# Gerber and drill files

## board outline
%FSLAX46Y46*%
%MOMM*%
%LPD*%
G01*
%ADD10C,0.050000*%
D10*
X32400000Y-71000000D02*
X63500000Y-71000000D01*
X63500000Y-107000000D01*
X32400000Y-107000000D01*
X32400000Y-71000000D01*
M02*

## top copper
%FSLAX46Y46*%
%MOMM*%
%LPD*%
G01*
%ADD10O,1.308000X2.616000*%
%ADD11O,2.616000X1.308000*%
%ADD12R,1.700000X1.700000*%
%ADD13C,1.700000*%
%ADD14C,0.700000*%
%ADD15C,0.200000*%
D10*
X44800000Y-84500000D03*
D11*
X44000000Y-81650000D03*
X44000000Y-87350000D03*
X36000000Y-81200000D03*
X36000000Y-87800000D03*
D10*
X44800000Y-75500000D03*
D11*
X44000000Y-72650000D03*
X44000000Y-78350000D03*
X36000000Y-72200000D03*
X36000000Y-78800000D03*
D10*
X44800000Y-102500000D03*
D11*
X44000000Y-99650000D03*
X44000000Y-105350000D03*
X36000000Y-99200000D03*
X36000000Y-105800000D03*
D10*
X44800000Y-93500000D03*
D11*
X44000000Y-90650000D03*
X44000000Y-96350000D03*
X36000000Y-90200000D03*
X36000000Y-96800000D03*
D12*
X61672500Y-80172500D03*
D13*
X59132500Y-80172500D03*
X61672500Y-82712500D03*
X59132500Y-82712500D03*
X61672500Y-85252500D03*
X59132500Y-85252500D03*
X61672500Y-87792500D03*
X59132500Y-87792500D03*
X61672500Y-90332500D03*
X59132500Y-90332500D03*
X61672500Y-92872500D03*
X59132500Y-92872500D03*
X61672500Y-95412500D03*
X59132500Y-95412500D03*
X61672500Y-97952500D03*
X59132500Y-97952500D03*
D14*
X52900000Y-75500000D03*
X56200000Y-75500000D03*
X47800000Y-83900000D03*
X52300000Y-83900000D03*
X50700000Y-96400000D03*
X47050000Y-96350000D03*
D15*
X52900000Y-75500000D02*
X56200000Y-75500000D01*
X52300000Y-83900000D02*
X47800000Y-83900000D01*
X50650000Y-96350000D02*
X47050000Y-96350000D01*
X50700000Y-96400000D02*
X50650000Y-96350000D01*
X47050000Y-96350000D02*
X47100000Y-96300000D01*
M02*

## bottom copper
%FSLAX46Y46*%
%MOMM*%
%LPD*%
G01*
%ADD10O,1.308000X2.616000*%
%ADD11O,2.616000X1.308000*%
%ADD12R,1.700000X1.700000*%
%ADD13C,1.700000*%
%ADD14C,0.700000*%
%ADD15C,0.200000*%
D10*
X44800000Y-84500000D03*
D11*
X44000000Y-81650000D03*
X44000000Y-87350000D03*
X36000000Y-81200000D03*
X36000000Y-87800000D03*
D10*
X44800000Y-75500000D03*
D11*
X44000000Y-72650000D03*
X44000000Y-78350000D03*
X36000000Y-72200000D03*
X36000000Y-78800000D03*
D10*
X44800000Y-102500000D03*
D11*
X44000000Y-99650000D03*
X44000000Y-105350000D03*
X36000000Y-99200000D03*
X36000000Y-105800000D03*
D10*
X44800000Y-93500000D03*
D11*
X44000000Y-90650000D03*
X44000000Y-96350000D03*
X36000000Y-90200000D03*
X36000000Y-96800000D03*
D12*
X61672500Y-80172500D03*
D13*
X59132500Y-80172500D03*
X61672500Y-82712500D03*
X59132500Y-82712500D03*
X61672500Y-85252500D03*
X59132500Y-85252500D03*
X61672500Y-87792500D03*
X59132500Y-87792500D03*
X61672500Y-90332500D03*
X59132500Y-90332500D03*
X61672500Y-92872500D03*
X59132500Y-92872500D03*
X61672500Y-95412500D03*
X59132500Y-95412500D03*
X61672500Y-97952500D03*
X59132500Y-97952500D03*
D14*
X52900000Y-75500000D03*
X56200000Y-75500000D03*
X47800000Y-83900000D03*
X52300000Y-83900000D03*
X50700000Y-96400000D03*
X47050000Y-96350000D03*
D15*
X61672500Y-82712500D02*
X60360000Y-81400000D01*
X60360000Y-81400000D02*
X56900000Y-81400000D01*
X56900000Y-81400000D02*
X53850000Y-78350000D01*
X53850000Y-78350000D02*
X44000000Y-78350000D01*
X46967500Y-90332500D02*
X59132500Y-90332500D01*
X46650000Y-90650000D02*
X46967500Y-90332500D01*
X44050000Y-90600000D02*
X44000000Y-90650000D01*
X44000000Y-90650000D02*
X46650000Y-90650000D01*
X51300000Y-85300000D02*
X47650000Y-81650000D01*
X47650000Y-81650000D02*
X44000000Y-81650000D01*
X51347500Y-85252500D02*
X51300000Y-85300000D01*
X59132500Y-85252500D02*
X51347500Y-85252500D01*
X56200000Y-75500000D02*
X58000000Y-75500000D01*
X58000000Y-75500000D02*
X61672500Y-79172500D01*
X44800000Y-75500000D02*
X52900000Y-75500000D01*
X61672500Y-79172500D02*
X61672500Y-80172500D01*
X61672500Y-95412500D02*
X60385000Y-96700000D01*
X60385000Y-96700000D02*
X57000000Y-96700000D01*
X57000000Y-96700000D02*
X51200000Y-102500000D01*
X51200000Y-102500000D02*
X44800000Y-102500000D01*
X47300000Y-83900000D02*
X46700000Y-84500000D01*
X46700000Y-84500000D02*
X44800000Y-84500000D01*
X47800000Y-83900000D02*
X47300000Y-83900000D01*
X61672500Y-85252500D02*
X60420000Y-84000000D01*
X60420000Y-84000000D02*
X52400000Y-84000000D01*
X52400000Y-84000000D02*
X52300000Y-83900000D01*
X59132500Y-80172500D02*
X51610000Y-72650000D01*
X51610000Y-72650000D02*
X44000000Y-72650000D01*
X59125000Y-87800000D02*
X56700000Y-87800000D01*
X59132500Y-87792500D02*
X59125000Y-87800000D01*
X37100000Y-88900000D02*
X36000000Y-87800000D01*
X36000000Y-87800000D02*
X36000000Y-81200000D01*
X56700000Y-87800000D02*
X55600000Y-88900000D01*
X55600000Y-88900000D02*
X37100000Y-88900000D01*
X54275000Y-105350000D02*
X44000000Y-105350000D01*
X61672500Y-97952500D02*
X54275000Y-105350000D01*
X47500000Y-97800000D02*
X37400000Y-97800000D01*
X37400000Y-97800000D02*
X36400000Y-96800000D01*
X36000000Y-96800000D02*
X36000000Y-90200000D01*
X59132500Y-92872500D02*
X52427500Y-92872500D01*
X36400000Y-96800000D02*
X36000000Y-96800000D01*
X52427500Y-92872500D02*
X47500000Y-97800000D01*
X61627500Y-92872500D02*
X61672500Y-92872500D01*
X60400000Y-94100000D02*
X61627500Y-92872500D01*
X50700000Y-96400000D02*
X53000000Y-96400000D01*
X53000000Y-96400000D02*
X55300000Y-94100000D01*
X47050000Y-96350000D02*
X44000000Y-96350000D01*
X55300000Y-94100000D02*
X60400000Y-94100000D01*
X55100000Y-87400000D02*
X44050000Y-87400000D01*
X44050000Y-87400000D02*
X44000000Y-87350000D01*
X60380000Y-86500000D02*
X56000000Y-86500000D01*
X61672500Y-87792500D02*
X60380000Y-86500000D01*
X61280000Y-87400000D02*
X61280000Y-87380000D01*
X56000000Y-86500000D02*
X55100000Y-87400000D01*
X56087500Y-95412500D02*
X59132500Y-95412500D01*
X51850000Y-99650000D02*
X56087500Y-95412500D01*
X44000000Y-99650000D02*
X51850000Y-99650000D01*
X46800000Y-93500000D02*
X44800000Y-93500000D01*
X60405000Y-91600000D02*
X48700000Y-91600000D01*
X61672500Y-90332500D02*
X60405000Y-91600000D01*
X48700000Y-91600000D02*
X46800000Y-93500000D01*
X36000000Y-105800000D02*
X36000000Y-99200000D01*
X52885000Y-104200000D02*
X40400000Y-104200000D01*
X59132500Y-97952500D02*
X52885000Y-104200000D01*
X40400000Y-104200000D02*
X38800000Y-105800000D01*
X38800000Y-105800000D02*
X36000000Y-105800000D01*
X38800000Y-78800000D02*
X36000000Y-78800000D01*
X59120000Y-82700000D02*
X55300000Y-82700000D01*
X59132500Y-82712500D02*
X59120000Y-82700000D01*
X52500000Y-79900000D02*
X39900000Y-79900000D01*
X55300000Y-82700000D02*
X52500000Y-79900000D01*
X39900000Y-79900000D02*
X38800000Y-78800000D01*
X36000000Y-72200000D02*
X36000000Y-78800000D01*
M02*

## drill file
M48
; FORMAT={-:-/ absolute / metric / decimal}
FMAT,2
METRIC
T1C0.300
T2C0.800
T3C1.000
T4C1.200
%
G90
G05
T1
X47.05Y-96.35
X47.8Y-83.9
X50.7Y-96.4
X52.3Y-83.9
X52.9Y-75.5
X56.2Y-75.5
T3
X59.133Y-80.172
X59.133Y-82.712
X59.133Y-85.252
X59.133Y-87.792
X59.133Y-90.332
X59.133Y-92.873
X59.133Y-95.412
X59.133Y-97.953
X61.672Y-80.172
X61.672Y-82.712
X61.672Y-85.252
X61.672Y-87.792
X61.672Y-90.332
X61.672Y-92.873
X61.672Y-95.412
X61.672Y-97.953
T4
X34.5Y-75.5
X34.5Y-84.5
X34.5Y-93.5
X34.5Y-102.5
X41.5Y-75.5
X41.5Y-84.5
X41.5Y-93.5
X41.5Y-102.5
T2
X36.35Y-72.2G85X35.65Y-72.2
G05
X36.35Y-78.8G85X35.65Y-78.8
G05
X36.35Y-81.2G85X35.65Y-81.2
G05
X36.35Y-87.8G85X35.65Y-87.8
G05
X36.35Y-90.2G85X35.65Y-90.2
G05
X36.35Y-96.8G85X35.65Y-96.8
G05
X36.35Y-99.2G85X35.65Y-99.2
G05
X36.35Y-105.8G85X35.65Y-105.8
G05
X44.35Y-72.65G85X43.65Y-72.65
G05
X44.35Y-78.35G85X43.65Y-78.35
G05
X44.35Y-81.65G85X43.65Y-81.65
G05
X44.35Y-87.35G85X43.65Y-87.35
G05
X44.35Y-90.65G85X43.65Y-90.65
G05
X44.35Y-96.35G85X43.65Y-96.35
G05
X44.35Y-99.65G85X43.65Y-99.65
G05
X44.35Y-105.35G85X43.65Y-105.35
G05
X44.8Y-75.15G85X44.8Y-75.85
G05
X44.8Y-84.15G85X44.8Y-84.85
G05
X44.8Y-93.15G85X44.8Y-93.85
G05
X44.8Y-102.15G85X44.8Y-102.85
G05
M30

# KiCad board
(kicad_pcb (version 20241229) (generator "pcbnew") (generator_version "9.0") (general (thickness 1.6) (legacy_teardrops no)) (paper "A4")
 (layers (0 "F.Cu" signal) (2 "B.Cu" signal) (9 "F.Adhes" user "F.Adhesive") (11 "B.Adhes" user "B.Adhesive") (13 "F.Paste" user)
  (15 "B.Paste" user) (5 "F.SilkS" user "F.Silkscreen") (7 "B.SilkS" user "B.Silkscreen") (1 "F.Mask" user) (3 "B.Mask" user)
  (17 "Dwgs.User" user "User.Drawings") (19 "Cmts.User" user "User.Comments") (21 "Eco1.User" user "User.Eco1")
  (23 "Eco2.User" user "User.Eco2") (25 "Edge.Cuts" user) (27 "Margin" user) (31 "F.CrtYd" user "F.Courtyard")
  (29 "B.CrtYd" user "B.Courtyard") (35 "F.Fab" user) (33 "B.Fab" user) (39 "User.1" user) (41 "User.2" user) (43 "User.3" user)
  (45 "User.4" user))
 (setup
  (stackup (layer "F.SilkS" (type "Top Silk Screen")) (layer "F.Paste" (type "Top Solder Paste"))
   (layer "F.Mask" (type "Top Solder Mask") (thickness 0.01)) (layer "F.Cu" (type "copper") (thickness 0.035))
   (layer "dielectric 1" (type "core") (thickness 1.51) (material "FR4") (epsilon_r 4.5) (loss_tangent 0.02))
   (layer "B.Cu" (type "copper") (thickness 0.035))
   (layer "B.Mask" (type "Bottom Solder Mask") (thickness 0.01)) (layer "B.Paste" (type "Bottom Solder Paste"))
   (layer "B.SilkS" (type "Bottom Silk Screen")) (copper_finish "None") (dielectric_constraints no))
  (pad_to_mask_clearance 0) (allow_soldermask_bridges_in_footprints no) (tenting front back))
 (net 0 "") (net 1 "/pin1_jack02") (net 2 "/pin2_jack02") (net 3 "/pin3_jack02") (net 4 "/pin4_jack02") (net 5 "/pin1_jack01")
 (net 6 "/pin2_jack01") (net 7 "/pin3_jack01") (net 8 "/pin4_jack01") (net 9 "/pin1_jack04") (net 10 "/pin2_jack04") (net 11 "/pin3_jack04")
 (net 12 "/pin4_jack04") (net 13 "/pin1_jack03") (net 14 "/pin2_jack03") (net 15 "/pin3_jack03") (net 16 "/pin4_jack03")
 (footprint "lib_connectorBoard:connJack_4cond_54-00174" (layer "F.Cu") (at 38 84.5 -90)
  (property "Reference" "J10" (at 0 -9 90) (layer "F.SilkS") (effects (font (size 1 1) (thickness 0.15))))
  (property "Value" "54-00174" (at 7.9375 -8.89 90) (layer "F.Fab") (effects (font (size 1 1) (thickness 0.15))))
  (pad "" np_thru_hole circle (at 0 -3.5 270) (size 1.2 1.2) (drill 1.2) (layers "*.Cu" "*.Mask"))
  (pad "" np_thru_hole circle (at 0 3.5 270) (size 1.2 1.2) (drill 1.2) (layers "*.Cu" "*.Mask"))
  (pad "1" thru_hole oval (at 0 -6.8 270) (size 2.616 1.308) (drill oval 1.5 0.8) (layers "*.Cu" "*.Mask") (remove_unused_layers no)
   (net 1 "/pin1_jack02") (solder_mask_margin 0.102))
  (pad "2" thru_hole oval (at -2.85 -6 270) (size 1.308 2.616) (drill oval 0.8 1.5) (layers "*.Cu" "*.Mask") (remove_unused_layers no)
   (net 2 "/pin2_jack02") (solder_mask_margin 0.102))
  (pad "3" thru_hole oval (at 2.85 -6 270) (size 1.308 2.616) (drill oval 0.8 1.5) (layers "*.Cu" "*.Mask") (remove_unused_layers no)
   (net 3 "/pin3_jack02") (solder_mask_margin 0.102))
  (pad "4_1" thru_hole oval (at -3.3 2 270) (size 1.308 2.616) (drill oval 0.8 1.5) (layers "*.Cu" "*.Mask") (remove_unused_layers no)
   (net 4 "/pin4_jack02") (solder_mask_margin 0.102))
  (pad "4_2" thru_hole oval (at 3.3 2 270) (size 1.308 2.616) (drill oval 0.8 1.5) (layers "*.Cu" "*.Mask") (remove_unused_layers no)
   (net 4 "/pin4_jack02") (solder_mask_margin 0.102)))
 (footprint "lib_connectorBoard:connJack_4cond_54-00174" (layer "F.Cu") (at 38 75.5 -90)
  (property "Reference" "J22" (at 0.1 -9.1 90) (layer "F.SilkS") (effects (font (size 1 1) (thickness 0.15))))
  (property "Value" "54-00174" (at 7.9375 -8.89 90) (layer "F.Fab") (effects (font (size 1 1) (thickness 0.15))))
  (pad "" np_thru_hole circle (at 0 -3.5 270) (size 1.2 1.2) (drill 1.2) (layers "*.Cu" "*.Mask"))
  (pad "" np_thru_hole circle (at 0 3.5 270) (size 1.2 1.2) (drill 1.2) (layers "*.Cu" "*.Mask"))
  (pad "1" thru_hole oval (at 0 -6.8 270) (size 2.616 1.308) (drill oval 1.5 0.8) (layers "*.Cu" "*.Mask") (remove_unused_layers no)
   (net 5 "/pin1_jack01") (solder_mask_margin 0.102))
  (pad "2" thru_hole oval (at -2.85 -6 270) (size 1.308 2.616) (drill oval 0.8 1.5) (layers "*.Cu" "*.Mask") (remove_unused_layers no)
   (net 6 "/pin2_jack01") (solder_mask_margin 0.102))
  (pad "3" thru_hole oval (at 2.85 -6 270) (size 1.308 2.616) (drill oval 0.8 1.5) (layers "*.Cu" "*.Mask") (remove_unused_layers no)
   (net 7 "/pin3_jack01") (solder_mask_margin 0.102))
  (pad "4_1" thru_hole oval (at -3.3 2 270) (size 1.308 2.616) (drill oval 0.8 1.5) (layers "*.Cu" "*.Mask") (remove_unused_layers no)
   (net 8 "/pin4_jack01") (solder_mask_margin 0.102))
  (pad "4_2" thru_hole oval (at 3.3 2 270) (size 1.308 2.616) (drill oval 0.8 1.5) (layers "*.Cu" "*.Mask") (remove_unused_layers no)
   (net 8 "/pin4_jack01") (solder_mask_margin 0.102)))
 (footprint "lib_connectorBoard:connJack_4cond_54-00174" (layer "F.Cu") (at 38 102.5 -90)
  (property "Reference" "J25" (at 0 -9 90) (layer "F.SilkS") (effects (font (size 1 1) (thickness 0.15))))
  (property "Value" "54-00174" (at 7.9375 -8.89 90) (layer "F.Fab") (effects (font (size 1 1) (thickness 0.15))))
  (pad "" np_thru_hole circle (at 0 -3.5 270) (size 1.2 1.2) (drill 1.2) (layers "*.Cu" "*.Mask"))
  (pad "" np_thru_hole circle (at 0 3.5 270) (size 1.2 1.2) (drill 1.2) (layers "*.Cu" "*.Mask"))
  (pad "1" thru_hole oval (at 0 -6.8 270) (size 2.616 1.308) (drill oval 1.5 0.8) (layers "*.Cu" "*.Mask") (remove_unused_layers no)
   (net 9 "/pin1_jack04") (solder_mask_margin 0.102))
  (pad "2" thru_hole oval (at -2.85 -6 270) (size 1.308 2.616) (drill oval 0.8 1.5) (layers "*.Cu" "*.Mask") (remove_unused_layers no)
   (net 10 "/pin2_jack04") (solder_mask_margin 0.102))
  (pad "3" thru_hole oval (at 2.85 -6 270) (size 1.308 2.616) (drill oval 0.8 1.5) (layers "*.Cu" "*.Mask") (remove_unused_layers no)
   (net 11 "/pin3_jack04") (solder_mask_margin 0.102))
  (pad "4_1" thru_hole oval (at -3.3 2 270) (size 1.308 2.616) (drill oval 0.8 1.5) (layers "*.Cu" "*.Mask") (remove_unused_layers no)
   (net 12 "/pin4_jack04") (solder_mask_margin 0.102))
  (pad "4_2" thru_hole oval (at 3.3 2 270) (size 1.308 2.616) (drill oval 0.8 1.5) (layers "*.Cu" "*.Mask") (remove_unused_layers no)
   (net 12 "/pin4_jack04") (solder_mask_margin 0.102)))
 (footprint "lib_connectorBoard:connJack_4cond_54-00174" (layer "F.Cu") (at 38 93.5 -90)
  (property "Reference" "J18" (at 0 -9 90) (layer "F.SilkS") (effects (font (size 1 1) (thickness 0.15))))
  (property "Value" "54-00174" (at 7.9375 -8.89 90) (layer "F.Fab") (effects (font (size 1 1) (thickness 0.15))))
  (pad "" np_thru_hole circle (at 0 -3.5 270) (size 1.2 1.2) (drill 1.2) (layers "*.Cu" "*.Mask"))
  (pad "" np_thru_hole circle (at 0 3.5 270) (size 1.2 1.2) (drill 1.2) (layers "*.Cu" "*.Mask"))
  (pad "1" thru_hole oval (at 0 -6.8 270) (size 2.616 1.308) (drill oval 1.5 0.8) (layers "*.Cu" "*.Mask") (remove_unused_layers no)
   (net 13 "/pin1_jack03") (solder_mask_margin 0.102))
  (pad "2" thru_hole oval (at -2.85 -6 270) (size 1.308 2.616) (drill oval 0.8 1.5) (layers "*.Cu" "*.Mask") (remove_unused_layers no)
   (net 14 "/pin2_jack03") (solder_mask_margin 0.102))
  (pad "3" thru_hole oval (at 2.85 -6 270) (size 1.308 2.616) (drill oval 0.8 1.5) (layers "*.Cu" "*.Mask") (remove_unused_layers no)
   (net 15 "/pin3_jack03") (solder_mask_margin 0.102))
  (pad "4_1" thru_hole oval (at -3.3 2 270) (size 1.308 2.616) (drill oval 0.8 1.5) (layers "*.Cu" "*.Mask") (remove_unused_layers no)
   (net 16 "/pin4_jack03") (solder_mask_margin 0.102))
  (pad "4_2" thru_hole oval (at 3.3 2 270) (size 1.308 2.616) (drill oval 0.8 1.5) (layers "*.Cu" "*.Mask") (remove_unused_layers no)
   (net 16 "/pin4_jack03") (solder_mask_margin 0.102)))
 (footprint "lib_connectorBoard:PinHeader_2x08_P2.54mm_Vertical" (layer "B.Cu") (at 63.4225 78.5025 180)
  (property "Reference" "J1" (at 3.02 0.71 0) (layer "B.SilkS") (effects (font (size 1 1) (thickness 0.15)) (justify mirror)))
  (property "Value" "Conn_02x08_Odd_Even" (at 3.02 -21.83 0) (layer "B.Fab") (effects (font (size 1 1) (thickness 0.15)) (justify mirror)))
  (pad "1" thru_hole rect (at 1.75 -1.67 180) (size 1.7 1.7) (drill 1) (layers "*.Cu" "*.Mask") (remove_unused_layers no)
   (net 5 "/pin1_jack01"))
  (pad "2" thru_hole circle (at 4.29 -1.67 180) (size 1.7 1.7) (drill 1) (layers "*.Cu" "*.Mask") (remove_unused_layers no)
   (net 6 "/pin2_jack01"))
  (pad "3" thru_hole circle (at 1.75 -4.21 180) (size 1.7 1.7) (drill 1) (layers "*.Cu" "*.Mask") (remove_unused_layers no)
   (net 7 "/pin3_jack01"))
  (pad "4" thru_hole circle (at 4.29 -4.21 180) (size 1.7 1.7) (drill 1) (layers "*.Cu" "*.Mask") (remove_unused_layers no)
   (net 8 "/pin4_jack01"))
  (pad "5" thru_hole circle (at 1.75 -6.75 180) (size 1.7 1.7) (drill 1) (layers "*.Cu" "*.Mask") (remove_unused_layers no)
   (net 1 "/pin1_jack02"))
  (pad "6" thru_hole circle (at 4.29 -6.75 180) (size 1.7 1.7) (drill 1) (layers "*.Cu" "*.Mask") (remove_unused_layers no)
   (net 2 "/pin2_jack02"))
  (pad "7" thru_hole circle (at 1.75 -9.29 180) (size 1.7 1.7) (drill 1) (layers "*.Cu" "*.Mask") (remove_unused_layers no)
   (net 3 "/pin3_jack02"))
  (pad "8" thru_hole circle (at 4.29 -9.29 180) (size 1.7 1.7) (drill 1) (layers "*.Cu" "*.Mask") (remove_unused_layers no)
   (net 4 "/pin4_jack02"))
  (pad "9" thru_hole circle (at 1.75 -11.83 180) (size 1.7 1.7) (drill 1) (layers "*.Cu" "*.Mask") (remove_unused_layers no)
   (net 13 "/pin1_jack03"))
  (pad "10" thru_hole circle (at 4.29 -11.83 180) (size 1.7 1.7) (drill 1) (layers "*.Cu" "*.Mask") (remove_unused_layers no)
   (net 14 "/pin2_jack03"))
  (pad "11" thru_hole circle (at 1.75 -14.37 180) (size 1.7 1.7) (drill 1) (layers "*.Cu" "*.Mask") (remove_unused_layers no)
   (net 15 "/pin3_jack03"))
  (pad "12" thru_hole circle (at 4.29 -14.37 180) (size 1.7 1.7) (drill 1) (layers "*.Cu" "*.Mask") (remove_unused_layers no)
   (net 16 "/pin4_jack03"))
  (pad "13" thru_hole circle (at 1.75 -16.91 180) (size 1.7 1.7) (drill 1) (layers "*.Cu" "*.Mask") (remove_unused_layers no)
   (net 9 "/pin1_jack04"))
  (pad "14" thru_hole circle (at 4.29 -16.91 180) (size 1.7 1.7) (drill 1) (layers "*.Cu" "*.Mask") (remove_unused_layers no)
   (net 10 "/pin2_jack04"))
  (pad "15" thru_hole circle (at 1.75 -19.45 180) (size 1.7 1.7) (drill 1) (layers "*.Cu" "*.Mask") (remove_unused_layers no)
   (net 11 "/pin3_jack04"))
  (pad "16" thru_hole circle (at 4.29 -19.45 180) (size 1.7 1.7) (drill 1) (layers "*.Cu" "*.Mask") (remove_unused_layers no)
   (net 12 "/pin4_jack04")))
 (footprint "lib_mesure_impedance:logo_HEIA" (layer "B.Cu") (at 48.8 77.9 -90)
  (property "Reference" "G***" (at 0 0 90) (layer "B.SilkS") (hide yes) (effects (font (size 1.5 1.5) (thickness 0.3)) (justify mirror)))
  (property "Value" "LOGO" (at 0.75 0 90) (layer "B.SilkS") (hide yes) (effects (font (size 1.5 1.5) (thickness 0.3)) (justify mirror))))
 (gr_rect (start 32.4 71) (end 63.5 107) (stroke (width 0.05) (type default)) (fill no) (layer "Edge.Cuts"))
 (segment (start 61.6725 82.7125) (end 60.36 81.4) (width 0.2) (layer "B.Cu") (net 7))
 (segment (start 60.36 81.4) (end 56.9 81.4) (width 0.2) (layer "B.Cu") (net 7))
 (segment (start 56.9 81.4) (end 53.85 78.35) (width 0.2) (layer "B.Cu") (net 7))
 (segment (start 53.85 78.35) (end 44 78.35) (width 0.2) (layer "B.Cu") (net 7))
 (segment (start 46.9675 90.3325) (end 59.1325 90.3325) (width 0.2) (layer "B.Cu") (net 14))
 (segment (start 46.65 90.65) (end 46.9675 90.3325) (width 0.2) (layer "B.Cu") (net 14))
 (segment (start 44.05 90.6) (end 44 90.65) (width 0.2) (layer "B.Cu") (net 14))
 (segment (start 44 90.65) (end 46.65 90.65) (width 0.2) (layer "B.Cu") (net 14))
 (segment (start 51.3 85.3) (end 47.65 81.65) (width 0.2) (layer "B.Cu") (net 2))
 (segment (start 47.65 81.65) (end 44 81.65) (width 0.2) (layer "B.Cu") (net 2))
 (segment (start 51.3475 85.2525) (end 51.3 85.3) (width 0.2) (layer "B.Cu") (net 2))
 (segment (start 59.1325 85.2525) (end 51.3475 85.2525) (width 0.2) (layer "B.Cu") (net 2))
 (segment (start 52.9 75.5) (end 56.2 75.5) (width 0.2) (layer "F.Cu") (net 5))
 (via (at 52.9 75.5) (size 0.7) (drill 0.3) (layers "F.Cu" "B.Cu") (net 5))
 (via (at 56.2 75.5) (size 0.7) (drill 0.3) (layers "F.Cu" "B.Cu") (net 5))
 (segment (start 56.2 75.5) (end 58 75.5) (width 0.2) (layer "B.Cu") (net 5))
 (segment (start 58 75.5) (end 61.6725 79.1725) (width 0.2) (layer "B.Cu") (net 5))
 (segment (start 44.8 75.5) (end 52.9 75.5) (width 0.2) (layer "B.Cu") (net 5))
 (segment (start 61.6725 79.1725) (end 61.6725 80.1725) (width 0.2) (layer "B.Cu") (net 5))
 (segment (start 61.6725 95.4125) (end 60.385 96.7) (width 0.2) (layer "B.Cu") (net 9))
 (segment (start 60.385 96.7) (end 57 96.7) (width 0.2) (layer "B.Cu") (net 9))
 (segment (start 57 96.7) (end 51.2 102.5) (width 0.2) (layer "B.Cu") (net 9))
 (segment (start 51.2 102.5) (end 44.8 102.5) (width 0.2) (layer "B.Cu") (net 9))
 (segment (start 52.3 83.9) (end 47.8 83.9) (width 0.2) (layer "F.Cu") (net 1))
 (via (at 47.8 83.9) (size 0.7) (drill 0.3) (layers "F.Cu" "B.Cu") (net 1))
 (via (at 52.3 83.9) (size 0.7) (drill 0.3) (layers "F.Cu" "B.Cu") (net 1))
 (segment (start 47.3 83.9) (end 46.7 84.5) (width 0.2) (layer "B.Cu") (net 1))
 (segment (start 46.7 84.5) (end 44.8 84.5) (width 0.2) (layer "B.Cu") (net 1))
 (segment (start 47.8 83.9) (end 47.3 83.9) (width 0.2) (layer "B.Cu") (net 1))
 (segment (start 61.6725 85.2525) (end 60.42 84) (width 0.2) (layer "B.Cu") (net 1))
 (segment (start 60.42 84) (end 52.4 84) (width 0.2) (layer "B.Cu") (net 1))
 (segment (start 52.4 84) (end 52.3 83.9) (width 0.2) (layer "B.Cu") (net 1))
 (segment (start 59.1325 80.1725) (end 51.61 72.65) (width 0.2) (layer "B.Cu") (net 6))
 (segment (start 51.61 72.65) (end 44 72.65) (width 0.2) (layer "B.Cu") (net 6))
 (segment (start 59.125 87.8) (end 56.7 87.8) (width 0.2) (layer "B.Cu") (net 4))
 (segment (start 59.1325 87.7925) (end 59.125 87.8) (width 0.2) (layer "B.Cu") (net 4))
 (segment (start 37.1 88.9) (end 36 87.8) (width 0.2) (layer "B.Cu") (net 4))
 (segment (start 36 87.8) (end 36 81.2) (width 0.2) (layer "B.Cu") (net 4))
 (segment (start 56.7 87.8) (end 55.6 88.9) (width 0.2) (layer "B.Cu") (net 4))
 (segment (start 55.6 88.9) (end 37.1 88.9) (width 0.2) (layer "B.Cu") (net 4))
 (segment (start 54.275 105.35) (end 44 105.35) (width 0.2) (layer "B.Cu") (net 11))
 (segment (start 61.6725 97.9525) (end 54.275 105.35) (width 0.2) (layer "B.Cu") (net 11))
 (segment (start 47.5 97.8) (end 37.4 97.8) (width 0.2) (layer "B.Cu") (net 16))
 (segment (start 37.4 97.8) (end 36.4 96.8) (width 0.2) (layer "B.Cu") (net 16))
 (segment (start 36 96.8) (end 36 90.2) (width 0.2) (layer "B.Cu") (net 16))
 (segment (start 59.1325 92.8725) (end 52.4275 92.8725) (width 0.2) (layer "B.Cu") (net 16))
 (segment (start 36.4 96.8) (end 36 96.8) (width 0.2) (layer "B.Cu") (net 16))
 (segment (start 52.4275 92.8725) (end 47.5 97.8) (width 0.2) (layer "B.Cu") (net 16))
 (segment (start 50.65 96.35) (end 47.05 96.35) (width 0.2) (layer "F.Cu") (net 15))
 (segment (start 50.7 96.4) (end 50.65 96.35) (width 0.2) (layer "F.Cu") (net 15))
 (segment (start 47.05 96.35) (end 47.1 96.3) (width 0.2) (layer "F.Cu") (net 15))
 (via (at 50.7 96.4) (size 0.7) (drill 0.3) (layers "F.Cu" "B.Cu") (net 15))
 (via (at 47.05 96.35) (size 0.7) (drill 0.3) (layers "F.Cu" "B.Cu") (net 15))
 (segment (start 61.6275 92.8725) (end 61.6725 92.8725) (width 0.2) (layer "B.Cu") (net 15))
 (segment (start 60.4 94.1) (end 61.6275 92.8725) (width 0.2) (layer "B.Cu") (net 15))
 (segment (start 50.7 96.4) (end 53 96.4) (width 0.2) (layer "B.Cu") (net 15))
 (segment (start 53 96.4) (end 55.3 94.1) (width 0.2) (layer "B.Cu") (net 15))
 (segment (start 47.05 96.35) (end 44 96.35) (width 0.2) (layer "B.Cu") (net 15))
 (segment (start 55.3 94.1) (end 60.4 94.1) (width 0.2) (layer "B.Cu") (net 15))
 (segment (start 55.1 87.4) (end 44.05 87.4) (width 0.2) (layer "B.Cu") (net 3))
 (segment (start 44.05 87.4) (end 44 87.35) (width 0.2) (layer "B.Cu") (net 3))
 (segment (start 60.38 86.5) (end 56 86.5) (width 0.2) (layer "B.Cu") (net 3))
 (segment (start 61.6725 87.7925) (end 60.38 86.5) (width 0.2) (layer "B.Cu") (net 3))
 (segment (start 61.28 87.4) (end 61.28 87.38) (width 0.2) (layer "B.Cu") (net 3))
 (segment (start 56 86.5) (end 55.1 87.4) (width 0.2) (layer "B.Cu") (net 3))
 (segment (start 56.0875 95.4125) (end 59.1325 95.4125) (width 0.2) (layer "B.Cu") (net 10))
 (segment (start 51.85 99.65) (end 56.0875 95.4125) (width 0.2) (layer "B.Cu") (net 10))
 (segment (start 44 99.65) (end 51.85 99.65) (width 0.2) (layer "B.Cu") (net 10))
 (segment (start 46.8 93.5) (end 44.8 93.5) (width 0.2) (layer "B.Cu") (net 13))
 (segment (start 60.405 91.6) (end 48.7 91.6) (width 0.2) (layer "B.Cu") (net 13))
 (segment (start 61.6725 90.3325) (end 60.405 91.6) (width 0.2) (layer "B.Cu") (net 13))
 (segment (start 48.7 91.6) (end 46.8 93.5) (width 0.2) (layer "B.Cu") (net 13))
 (segment (start 36 105.8) (end 36 99.2) (width 0.2) (layer "B.Cu") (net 12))
 (segment (start 52.885 104.2) (end 40.4 104.2) (width 0.2) (layer "B.Cu") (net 12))
 (segment (start 59.1325 97.9525) (end 52.885 104.2) (width 0.2) (layer "B.Cu") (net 12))
 (segment (start 40.4 104.2) (end 38.8 105.8) (width 0.2) (layer "B.Cu") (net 12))
 (segment (start 38.8 105.8) (end 36 105.8) (width 0.2) (layer "B.Cu") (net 12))
 (segment (start 38.8 78.8) (end 36 78.8) (width 0.2) (layer "B.Cu") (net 8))
 (segment (start 59.12 82.7) (end 55.3 82.7) (width 0.2) (layer "B.Cu") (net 8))
 (segment (start 59.1325 82.7125) (end 59.12 82.7) (width 0.2) (layer "B.Cu") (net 8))
 (segment (start 52.5 79.9) (end 39.9 79.9) (width 0.2) (layer "B.Cu") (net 8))
 (segment (start 55.3 82.7) (end 52.5 79.9) (width 0.2) (layer "B.Cu") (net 8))
 (segment (start 39.9 79.9) (end 38.8 78.8) (width 0.2) (layer "B.Cu") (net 8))
 (segment (start 36 72.2) (end 36 78.8) (width 0.2) (layer "B.Cu") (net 8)))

